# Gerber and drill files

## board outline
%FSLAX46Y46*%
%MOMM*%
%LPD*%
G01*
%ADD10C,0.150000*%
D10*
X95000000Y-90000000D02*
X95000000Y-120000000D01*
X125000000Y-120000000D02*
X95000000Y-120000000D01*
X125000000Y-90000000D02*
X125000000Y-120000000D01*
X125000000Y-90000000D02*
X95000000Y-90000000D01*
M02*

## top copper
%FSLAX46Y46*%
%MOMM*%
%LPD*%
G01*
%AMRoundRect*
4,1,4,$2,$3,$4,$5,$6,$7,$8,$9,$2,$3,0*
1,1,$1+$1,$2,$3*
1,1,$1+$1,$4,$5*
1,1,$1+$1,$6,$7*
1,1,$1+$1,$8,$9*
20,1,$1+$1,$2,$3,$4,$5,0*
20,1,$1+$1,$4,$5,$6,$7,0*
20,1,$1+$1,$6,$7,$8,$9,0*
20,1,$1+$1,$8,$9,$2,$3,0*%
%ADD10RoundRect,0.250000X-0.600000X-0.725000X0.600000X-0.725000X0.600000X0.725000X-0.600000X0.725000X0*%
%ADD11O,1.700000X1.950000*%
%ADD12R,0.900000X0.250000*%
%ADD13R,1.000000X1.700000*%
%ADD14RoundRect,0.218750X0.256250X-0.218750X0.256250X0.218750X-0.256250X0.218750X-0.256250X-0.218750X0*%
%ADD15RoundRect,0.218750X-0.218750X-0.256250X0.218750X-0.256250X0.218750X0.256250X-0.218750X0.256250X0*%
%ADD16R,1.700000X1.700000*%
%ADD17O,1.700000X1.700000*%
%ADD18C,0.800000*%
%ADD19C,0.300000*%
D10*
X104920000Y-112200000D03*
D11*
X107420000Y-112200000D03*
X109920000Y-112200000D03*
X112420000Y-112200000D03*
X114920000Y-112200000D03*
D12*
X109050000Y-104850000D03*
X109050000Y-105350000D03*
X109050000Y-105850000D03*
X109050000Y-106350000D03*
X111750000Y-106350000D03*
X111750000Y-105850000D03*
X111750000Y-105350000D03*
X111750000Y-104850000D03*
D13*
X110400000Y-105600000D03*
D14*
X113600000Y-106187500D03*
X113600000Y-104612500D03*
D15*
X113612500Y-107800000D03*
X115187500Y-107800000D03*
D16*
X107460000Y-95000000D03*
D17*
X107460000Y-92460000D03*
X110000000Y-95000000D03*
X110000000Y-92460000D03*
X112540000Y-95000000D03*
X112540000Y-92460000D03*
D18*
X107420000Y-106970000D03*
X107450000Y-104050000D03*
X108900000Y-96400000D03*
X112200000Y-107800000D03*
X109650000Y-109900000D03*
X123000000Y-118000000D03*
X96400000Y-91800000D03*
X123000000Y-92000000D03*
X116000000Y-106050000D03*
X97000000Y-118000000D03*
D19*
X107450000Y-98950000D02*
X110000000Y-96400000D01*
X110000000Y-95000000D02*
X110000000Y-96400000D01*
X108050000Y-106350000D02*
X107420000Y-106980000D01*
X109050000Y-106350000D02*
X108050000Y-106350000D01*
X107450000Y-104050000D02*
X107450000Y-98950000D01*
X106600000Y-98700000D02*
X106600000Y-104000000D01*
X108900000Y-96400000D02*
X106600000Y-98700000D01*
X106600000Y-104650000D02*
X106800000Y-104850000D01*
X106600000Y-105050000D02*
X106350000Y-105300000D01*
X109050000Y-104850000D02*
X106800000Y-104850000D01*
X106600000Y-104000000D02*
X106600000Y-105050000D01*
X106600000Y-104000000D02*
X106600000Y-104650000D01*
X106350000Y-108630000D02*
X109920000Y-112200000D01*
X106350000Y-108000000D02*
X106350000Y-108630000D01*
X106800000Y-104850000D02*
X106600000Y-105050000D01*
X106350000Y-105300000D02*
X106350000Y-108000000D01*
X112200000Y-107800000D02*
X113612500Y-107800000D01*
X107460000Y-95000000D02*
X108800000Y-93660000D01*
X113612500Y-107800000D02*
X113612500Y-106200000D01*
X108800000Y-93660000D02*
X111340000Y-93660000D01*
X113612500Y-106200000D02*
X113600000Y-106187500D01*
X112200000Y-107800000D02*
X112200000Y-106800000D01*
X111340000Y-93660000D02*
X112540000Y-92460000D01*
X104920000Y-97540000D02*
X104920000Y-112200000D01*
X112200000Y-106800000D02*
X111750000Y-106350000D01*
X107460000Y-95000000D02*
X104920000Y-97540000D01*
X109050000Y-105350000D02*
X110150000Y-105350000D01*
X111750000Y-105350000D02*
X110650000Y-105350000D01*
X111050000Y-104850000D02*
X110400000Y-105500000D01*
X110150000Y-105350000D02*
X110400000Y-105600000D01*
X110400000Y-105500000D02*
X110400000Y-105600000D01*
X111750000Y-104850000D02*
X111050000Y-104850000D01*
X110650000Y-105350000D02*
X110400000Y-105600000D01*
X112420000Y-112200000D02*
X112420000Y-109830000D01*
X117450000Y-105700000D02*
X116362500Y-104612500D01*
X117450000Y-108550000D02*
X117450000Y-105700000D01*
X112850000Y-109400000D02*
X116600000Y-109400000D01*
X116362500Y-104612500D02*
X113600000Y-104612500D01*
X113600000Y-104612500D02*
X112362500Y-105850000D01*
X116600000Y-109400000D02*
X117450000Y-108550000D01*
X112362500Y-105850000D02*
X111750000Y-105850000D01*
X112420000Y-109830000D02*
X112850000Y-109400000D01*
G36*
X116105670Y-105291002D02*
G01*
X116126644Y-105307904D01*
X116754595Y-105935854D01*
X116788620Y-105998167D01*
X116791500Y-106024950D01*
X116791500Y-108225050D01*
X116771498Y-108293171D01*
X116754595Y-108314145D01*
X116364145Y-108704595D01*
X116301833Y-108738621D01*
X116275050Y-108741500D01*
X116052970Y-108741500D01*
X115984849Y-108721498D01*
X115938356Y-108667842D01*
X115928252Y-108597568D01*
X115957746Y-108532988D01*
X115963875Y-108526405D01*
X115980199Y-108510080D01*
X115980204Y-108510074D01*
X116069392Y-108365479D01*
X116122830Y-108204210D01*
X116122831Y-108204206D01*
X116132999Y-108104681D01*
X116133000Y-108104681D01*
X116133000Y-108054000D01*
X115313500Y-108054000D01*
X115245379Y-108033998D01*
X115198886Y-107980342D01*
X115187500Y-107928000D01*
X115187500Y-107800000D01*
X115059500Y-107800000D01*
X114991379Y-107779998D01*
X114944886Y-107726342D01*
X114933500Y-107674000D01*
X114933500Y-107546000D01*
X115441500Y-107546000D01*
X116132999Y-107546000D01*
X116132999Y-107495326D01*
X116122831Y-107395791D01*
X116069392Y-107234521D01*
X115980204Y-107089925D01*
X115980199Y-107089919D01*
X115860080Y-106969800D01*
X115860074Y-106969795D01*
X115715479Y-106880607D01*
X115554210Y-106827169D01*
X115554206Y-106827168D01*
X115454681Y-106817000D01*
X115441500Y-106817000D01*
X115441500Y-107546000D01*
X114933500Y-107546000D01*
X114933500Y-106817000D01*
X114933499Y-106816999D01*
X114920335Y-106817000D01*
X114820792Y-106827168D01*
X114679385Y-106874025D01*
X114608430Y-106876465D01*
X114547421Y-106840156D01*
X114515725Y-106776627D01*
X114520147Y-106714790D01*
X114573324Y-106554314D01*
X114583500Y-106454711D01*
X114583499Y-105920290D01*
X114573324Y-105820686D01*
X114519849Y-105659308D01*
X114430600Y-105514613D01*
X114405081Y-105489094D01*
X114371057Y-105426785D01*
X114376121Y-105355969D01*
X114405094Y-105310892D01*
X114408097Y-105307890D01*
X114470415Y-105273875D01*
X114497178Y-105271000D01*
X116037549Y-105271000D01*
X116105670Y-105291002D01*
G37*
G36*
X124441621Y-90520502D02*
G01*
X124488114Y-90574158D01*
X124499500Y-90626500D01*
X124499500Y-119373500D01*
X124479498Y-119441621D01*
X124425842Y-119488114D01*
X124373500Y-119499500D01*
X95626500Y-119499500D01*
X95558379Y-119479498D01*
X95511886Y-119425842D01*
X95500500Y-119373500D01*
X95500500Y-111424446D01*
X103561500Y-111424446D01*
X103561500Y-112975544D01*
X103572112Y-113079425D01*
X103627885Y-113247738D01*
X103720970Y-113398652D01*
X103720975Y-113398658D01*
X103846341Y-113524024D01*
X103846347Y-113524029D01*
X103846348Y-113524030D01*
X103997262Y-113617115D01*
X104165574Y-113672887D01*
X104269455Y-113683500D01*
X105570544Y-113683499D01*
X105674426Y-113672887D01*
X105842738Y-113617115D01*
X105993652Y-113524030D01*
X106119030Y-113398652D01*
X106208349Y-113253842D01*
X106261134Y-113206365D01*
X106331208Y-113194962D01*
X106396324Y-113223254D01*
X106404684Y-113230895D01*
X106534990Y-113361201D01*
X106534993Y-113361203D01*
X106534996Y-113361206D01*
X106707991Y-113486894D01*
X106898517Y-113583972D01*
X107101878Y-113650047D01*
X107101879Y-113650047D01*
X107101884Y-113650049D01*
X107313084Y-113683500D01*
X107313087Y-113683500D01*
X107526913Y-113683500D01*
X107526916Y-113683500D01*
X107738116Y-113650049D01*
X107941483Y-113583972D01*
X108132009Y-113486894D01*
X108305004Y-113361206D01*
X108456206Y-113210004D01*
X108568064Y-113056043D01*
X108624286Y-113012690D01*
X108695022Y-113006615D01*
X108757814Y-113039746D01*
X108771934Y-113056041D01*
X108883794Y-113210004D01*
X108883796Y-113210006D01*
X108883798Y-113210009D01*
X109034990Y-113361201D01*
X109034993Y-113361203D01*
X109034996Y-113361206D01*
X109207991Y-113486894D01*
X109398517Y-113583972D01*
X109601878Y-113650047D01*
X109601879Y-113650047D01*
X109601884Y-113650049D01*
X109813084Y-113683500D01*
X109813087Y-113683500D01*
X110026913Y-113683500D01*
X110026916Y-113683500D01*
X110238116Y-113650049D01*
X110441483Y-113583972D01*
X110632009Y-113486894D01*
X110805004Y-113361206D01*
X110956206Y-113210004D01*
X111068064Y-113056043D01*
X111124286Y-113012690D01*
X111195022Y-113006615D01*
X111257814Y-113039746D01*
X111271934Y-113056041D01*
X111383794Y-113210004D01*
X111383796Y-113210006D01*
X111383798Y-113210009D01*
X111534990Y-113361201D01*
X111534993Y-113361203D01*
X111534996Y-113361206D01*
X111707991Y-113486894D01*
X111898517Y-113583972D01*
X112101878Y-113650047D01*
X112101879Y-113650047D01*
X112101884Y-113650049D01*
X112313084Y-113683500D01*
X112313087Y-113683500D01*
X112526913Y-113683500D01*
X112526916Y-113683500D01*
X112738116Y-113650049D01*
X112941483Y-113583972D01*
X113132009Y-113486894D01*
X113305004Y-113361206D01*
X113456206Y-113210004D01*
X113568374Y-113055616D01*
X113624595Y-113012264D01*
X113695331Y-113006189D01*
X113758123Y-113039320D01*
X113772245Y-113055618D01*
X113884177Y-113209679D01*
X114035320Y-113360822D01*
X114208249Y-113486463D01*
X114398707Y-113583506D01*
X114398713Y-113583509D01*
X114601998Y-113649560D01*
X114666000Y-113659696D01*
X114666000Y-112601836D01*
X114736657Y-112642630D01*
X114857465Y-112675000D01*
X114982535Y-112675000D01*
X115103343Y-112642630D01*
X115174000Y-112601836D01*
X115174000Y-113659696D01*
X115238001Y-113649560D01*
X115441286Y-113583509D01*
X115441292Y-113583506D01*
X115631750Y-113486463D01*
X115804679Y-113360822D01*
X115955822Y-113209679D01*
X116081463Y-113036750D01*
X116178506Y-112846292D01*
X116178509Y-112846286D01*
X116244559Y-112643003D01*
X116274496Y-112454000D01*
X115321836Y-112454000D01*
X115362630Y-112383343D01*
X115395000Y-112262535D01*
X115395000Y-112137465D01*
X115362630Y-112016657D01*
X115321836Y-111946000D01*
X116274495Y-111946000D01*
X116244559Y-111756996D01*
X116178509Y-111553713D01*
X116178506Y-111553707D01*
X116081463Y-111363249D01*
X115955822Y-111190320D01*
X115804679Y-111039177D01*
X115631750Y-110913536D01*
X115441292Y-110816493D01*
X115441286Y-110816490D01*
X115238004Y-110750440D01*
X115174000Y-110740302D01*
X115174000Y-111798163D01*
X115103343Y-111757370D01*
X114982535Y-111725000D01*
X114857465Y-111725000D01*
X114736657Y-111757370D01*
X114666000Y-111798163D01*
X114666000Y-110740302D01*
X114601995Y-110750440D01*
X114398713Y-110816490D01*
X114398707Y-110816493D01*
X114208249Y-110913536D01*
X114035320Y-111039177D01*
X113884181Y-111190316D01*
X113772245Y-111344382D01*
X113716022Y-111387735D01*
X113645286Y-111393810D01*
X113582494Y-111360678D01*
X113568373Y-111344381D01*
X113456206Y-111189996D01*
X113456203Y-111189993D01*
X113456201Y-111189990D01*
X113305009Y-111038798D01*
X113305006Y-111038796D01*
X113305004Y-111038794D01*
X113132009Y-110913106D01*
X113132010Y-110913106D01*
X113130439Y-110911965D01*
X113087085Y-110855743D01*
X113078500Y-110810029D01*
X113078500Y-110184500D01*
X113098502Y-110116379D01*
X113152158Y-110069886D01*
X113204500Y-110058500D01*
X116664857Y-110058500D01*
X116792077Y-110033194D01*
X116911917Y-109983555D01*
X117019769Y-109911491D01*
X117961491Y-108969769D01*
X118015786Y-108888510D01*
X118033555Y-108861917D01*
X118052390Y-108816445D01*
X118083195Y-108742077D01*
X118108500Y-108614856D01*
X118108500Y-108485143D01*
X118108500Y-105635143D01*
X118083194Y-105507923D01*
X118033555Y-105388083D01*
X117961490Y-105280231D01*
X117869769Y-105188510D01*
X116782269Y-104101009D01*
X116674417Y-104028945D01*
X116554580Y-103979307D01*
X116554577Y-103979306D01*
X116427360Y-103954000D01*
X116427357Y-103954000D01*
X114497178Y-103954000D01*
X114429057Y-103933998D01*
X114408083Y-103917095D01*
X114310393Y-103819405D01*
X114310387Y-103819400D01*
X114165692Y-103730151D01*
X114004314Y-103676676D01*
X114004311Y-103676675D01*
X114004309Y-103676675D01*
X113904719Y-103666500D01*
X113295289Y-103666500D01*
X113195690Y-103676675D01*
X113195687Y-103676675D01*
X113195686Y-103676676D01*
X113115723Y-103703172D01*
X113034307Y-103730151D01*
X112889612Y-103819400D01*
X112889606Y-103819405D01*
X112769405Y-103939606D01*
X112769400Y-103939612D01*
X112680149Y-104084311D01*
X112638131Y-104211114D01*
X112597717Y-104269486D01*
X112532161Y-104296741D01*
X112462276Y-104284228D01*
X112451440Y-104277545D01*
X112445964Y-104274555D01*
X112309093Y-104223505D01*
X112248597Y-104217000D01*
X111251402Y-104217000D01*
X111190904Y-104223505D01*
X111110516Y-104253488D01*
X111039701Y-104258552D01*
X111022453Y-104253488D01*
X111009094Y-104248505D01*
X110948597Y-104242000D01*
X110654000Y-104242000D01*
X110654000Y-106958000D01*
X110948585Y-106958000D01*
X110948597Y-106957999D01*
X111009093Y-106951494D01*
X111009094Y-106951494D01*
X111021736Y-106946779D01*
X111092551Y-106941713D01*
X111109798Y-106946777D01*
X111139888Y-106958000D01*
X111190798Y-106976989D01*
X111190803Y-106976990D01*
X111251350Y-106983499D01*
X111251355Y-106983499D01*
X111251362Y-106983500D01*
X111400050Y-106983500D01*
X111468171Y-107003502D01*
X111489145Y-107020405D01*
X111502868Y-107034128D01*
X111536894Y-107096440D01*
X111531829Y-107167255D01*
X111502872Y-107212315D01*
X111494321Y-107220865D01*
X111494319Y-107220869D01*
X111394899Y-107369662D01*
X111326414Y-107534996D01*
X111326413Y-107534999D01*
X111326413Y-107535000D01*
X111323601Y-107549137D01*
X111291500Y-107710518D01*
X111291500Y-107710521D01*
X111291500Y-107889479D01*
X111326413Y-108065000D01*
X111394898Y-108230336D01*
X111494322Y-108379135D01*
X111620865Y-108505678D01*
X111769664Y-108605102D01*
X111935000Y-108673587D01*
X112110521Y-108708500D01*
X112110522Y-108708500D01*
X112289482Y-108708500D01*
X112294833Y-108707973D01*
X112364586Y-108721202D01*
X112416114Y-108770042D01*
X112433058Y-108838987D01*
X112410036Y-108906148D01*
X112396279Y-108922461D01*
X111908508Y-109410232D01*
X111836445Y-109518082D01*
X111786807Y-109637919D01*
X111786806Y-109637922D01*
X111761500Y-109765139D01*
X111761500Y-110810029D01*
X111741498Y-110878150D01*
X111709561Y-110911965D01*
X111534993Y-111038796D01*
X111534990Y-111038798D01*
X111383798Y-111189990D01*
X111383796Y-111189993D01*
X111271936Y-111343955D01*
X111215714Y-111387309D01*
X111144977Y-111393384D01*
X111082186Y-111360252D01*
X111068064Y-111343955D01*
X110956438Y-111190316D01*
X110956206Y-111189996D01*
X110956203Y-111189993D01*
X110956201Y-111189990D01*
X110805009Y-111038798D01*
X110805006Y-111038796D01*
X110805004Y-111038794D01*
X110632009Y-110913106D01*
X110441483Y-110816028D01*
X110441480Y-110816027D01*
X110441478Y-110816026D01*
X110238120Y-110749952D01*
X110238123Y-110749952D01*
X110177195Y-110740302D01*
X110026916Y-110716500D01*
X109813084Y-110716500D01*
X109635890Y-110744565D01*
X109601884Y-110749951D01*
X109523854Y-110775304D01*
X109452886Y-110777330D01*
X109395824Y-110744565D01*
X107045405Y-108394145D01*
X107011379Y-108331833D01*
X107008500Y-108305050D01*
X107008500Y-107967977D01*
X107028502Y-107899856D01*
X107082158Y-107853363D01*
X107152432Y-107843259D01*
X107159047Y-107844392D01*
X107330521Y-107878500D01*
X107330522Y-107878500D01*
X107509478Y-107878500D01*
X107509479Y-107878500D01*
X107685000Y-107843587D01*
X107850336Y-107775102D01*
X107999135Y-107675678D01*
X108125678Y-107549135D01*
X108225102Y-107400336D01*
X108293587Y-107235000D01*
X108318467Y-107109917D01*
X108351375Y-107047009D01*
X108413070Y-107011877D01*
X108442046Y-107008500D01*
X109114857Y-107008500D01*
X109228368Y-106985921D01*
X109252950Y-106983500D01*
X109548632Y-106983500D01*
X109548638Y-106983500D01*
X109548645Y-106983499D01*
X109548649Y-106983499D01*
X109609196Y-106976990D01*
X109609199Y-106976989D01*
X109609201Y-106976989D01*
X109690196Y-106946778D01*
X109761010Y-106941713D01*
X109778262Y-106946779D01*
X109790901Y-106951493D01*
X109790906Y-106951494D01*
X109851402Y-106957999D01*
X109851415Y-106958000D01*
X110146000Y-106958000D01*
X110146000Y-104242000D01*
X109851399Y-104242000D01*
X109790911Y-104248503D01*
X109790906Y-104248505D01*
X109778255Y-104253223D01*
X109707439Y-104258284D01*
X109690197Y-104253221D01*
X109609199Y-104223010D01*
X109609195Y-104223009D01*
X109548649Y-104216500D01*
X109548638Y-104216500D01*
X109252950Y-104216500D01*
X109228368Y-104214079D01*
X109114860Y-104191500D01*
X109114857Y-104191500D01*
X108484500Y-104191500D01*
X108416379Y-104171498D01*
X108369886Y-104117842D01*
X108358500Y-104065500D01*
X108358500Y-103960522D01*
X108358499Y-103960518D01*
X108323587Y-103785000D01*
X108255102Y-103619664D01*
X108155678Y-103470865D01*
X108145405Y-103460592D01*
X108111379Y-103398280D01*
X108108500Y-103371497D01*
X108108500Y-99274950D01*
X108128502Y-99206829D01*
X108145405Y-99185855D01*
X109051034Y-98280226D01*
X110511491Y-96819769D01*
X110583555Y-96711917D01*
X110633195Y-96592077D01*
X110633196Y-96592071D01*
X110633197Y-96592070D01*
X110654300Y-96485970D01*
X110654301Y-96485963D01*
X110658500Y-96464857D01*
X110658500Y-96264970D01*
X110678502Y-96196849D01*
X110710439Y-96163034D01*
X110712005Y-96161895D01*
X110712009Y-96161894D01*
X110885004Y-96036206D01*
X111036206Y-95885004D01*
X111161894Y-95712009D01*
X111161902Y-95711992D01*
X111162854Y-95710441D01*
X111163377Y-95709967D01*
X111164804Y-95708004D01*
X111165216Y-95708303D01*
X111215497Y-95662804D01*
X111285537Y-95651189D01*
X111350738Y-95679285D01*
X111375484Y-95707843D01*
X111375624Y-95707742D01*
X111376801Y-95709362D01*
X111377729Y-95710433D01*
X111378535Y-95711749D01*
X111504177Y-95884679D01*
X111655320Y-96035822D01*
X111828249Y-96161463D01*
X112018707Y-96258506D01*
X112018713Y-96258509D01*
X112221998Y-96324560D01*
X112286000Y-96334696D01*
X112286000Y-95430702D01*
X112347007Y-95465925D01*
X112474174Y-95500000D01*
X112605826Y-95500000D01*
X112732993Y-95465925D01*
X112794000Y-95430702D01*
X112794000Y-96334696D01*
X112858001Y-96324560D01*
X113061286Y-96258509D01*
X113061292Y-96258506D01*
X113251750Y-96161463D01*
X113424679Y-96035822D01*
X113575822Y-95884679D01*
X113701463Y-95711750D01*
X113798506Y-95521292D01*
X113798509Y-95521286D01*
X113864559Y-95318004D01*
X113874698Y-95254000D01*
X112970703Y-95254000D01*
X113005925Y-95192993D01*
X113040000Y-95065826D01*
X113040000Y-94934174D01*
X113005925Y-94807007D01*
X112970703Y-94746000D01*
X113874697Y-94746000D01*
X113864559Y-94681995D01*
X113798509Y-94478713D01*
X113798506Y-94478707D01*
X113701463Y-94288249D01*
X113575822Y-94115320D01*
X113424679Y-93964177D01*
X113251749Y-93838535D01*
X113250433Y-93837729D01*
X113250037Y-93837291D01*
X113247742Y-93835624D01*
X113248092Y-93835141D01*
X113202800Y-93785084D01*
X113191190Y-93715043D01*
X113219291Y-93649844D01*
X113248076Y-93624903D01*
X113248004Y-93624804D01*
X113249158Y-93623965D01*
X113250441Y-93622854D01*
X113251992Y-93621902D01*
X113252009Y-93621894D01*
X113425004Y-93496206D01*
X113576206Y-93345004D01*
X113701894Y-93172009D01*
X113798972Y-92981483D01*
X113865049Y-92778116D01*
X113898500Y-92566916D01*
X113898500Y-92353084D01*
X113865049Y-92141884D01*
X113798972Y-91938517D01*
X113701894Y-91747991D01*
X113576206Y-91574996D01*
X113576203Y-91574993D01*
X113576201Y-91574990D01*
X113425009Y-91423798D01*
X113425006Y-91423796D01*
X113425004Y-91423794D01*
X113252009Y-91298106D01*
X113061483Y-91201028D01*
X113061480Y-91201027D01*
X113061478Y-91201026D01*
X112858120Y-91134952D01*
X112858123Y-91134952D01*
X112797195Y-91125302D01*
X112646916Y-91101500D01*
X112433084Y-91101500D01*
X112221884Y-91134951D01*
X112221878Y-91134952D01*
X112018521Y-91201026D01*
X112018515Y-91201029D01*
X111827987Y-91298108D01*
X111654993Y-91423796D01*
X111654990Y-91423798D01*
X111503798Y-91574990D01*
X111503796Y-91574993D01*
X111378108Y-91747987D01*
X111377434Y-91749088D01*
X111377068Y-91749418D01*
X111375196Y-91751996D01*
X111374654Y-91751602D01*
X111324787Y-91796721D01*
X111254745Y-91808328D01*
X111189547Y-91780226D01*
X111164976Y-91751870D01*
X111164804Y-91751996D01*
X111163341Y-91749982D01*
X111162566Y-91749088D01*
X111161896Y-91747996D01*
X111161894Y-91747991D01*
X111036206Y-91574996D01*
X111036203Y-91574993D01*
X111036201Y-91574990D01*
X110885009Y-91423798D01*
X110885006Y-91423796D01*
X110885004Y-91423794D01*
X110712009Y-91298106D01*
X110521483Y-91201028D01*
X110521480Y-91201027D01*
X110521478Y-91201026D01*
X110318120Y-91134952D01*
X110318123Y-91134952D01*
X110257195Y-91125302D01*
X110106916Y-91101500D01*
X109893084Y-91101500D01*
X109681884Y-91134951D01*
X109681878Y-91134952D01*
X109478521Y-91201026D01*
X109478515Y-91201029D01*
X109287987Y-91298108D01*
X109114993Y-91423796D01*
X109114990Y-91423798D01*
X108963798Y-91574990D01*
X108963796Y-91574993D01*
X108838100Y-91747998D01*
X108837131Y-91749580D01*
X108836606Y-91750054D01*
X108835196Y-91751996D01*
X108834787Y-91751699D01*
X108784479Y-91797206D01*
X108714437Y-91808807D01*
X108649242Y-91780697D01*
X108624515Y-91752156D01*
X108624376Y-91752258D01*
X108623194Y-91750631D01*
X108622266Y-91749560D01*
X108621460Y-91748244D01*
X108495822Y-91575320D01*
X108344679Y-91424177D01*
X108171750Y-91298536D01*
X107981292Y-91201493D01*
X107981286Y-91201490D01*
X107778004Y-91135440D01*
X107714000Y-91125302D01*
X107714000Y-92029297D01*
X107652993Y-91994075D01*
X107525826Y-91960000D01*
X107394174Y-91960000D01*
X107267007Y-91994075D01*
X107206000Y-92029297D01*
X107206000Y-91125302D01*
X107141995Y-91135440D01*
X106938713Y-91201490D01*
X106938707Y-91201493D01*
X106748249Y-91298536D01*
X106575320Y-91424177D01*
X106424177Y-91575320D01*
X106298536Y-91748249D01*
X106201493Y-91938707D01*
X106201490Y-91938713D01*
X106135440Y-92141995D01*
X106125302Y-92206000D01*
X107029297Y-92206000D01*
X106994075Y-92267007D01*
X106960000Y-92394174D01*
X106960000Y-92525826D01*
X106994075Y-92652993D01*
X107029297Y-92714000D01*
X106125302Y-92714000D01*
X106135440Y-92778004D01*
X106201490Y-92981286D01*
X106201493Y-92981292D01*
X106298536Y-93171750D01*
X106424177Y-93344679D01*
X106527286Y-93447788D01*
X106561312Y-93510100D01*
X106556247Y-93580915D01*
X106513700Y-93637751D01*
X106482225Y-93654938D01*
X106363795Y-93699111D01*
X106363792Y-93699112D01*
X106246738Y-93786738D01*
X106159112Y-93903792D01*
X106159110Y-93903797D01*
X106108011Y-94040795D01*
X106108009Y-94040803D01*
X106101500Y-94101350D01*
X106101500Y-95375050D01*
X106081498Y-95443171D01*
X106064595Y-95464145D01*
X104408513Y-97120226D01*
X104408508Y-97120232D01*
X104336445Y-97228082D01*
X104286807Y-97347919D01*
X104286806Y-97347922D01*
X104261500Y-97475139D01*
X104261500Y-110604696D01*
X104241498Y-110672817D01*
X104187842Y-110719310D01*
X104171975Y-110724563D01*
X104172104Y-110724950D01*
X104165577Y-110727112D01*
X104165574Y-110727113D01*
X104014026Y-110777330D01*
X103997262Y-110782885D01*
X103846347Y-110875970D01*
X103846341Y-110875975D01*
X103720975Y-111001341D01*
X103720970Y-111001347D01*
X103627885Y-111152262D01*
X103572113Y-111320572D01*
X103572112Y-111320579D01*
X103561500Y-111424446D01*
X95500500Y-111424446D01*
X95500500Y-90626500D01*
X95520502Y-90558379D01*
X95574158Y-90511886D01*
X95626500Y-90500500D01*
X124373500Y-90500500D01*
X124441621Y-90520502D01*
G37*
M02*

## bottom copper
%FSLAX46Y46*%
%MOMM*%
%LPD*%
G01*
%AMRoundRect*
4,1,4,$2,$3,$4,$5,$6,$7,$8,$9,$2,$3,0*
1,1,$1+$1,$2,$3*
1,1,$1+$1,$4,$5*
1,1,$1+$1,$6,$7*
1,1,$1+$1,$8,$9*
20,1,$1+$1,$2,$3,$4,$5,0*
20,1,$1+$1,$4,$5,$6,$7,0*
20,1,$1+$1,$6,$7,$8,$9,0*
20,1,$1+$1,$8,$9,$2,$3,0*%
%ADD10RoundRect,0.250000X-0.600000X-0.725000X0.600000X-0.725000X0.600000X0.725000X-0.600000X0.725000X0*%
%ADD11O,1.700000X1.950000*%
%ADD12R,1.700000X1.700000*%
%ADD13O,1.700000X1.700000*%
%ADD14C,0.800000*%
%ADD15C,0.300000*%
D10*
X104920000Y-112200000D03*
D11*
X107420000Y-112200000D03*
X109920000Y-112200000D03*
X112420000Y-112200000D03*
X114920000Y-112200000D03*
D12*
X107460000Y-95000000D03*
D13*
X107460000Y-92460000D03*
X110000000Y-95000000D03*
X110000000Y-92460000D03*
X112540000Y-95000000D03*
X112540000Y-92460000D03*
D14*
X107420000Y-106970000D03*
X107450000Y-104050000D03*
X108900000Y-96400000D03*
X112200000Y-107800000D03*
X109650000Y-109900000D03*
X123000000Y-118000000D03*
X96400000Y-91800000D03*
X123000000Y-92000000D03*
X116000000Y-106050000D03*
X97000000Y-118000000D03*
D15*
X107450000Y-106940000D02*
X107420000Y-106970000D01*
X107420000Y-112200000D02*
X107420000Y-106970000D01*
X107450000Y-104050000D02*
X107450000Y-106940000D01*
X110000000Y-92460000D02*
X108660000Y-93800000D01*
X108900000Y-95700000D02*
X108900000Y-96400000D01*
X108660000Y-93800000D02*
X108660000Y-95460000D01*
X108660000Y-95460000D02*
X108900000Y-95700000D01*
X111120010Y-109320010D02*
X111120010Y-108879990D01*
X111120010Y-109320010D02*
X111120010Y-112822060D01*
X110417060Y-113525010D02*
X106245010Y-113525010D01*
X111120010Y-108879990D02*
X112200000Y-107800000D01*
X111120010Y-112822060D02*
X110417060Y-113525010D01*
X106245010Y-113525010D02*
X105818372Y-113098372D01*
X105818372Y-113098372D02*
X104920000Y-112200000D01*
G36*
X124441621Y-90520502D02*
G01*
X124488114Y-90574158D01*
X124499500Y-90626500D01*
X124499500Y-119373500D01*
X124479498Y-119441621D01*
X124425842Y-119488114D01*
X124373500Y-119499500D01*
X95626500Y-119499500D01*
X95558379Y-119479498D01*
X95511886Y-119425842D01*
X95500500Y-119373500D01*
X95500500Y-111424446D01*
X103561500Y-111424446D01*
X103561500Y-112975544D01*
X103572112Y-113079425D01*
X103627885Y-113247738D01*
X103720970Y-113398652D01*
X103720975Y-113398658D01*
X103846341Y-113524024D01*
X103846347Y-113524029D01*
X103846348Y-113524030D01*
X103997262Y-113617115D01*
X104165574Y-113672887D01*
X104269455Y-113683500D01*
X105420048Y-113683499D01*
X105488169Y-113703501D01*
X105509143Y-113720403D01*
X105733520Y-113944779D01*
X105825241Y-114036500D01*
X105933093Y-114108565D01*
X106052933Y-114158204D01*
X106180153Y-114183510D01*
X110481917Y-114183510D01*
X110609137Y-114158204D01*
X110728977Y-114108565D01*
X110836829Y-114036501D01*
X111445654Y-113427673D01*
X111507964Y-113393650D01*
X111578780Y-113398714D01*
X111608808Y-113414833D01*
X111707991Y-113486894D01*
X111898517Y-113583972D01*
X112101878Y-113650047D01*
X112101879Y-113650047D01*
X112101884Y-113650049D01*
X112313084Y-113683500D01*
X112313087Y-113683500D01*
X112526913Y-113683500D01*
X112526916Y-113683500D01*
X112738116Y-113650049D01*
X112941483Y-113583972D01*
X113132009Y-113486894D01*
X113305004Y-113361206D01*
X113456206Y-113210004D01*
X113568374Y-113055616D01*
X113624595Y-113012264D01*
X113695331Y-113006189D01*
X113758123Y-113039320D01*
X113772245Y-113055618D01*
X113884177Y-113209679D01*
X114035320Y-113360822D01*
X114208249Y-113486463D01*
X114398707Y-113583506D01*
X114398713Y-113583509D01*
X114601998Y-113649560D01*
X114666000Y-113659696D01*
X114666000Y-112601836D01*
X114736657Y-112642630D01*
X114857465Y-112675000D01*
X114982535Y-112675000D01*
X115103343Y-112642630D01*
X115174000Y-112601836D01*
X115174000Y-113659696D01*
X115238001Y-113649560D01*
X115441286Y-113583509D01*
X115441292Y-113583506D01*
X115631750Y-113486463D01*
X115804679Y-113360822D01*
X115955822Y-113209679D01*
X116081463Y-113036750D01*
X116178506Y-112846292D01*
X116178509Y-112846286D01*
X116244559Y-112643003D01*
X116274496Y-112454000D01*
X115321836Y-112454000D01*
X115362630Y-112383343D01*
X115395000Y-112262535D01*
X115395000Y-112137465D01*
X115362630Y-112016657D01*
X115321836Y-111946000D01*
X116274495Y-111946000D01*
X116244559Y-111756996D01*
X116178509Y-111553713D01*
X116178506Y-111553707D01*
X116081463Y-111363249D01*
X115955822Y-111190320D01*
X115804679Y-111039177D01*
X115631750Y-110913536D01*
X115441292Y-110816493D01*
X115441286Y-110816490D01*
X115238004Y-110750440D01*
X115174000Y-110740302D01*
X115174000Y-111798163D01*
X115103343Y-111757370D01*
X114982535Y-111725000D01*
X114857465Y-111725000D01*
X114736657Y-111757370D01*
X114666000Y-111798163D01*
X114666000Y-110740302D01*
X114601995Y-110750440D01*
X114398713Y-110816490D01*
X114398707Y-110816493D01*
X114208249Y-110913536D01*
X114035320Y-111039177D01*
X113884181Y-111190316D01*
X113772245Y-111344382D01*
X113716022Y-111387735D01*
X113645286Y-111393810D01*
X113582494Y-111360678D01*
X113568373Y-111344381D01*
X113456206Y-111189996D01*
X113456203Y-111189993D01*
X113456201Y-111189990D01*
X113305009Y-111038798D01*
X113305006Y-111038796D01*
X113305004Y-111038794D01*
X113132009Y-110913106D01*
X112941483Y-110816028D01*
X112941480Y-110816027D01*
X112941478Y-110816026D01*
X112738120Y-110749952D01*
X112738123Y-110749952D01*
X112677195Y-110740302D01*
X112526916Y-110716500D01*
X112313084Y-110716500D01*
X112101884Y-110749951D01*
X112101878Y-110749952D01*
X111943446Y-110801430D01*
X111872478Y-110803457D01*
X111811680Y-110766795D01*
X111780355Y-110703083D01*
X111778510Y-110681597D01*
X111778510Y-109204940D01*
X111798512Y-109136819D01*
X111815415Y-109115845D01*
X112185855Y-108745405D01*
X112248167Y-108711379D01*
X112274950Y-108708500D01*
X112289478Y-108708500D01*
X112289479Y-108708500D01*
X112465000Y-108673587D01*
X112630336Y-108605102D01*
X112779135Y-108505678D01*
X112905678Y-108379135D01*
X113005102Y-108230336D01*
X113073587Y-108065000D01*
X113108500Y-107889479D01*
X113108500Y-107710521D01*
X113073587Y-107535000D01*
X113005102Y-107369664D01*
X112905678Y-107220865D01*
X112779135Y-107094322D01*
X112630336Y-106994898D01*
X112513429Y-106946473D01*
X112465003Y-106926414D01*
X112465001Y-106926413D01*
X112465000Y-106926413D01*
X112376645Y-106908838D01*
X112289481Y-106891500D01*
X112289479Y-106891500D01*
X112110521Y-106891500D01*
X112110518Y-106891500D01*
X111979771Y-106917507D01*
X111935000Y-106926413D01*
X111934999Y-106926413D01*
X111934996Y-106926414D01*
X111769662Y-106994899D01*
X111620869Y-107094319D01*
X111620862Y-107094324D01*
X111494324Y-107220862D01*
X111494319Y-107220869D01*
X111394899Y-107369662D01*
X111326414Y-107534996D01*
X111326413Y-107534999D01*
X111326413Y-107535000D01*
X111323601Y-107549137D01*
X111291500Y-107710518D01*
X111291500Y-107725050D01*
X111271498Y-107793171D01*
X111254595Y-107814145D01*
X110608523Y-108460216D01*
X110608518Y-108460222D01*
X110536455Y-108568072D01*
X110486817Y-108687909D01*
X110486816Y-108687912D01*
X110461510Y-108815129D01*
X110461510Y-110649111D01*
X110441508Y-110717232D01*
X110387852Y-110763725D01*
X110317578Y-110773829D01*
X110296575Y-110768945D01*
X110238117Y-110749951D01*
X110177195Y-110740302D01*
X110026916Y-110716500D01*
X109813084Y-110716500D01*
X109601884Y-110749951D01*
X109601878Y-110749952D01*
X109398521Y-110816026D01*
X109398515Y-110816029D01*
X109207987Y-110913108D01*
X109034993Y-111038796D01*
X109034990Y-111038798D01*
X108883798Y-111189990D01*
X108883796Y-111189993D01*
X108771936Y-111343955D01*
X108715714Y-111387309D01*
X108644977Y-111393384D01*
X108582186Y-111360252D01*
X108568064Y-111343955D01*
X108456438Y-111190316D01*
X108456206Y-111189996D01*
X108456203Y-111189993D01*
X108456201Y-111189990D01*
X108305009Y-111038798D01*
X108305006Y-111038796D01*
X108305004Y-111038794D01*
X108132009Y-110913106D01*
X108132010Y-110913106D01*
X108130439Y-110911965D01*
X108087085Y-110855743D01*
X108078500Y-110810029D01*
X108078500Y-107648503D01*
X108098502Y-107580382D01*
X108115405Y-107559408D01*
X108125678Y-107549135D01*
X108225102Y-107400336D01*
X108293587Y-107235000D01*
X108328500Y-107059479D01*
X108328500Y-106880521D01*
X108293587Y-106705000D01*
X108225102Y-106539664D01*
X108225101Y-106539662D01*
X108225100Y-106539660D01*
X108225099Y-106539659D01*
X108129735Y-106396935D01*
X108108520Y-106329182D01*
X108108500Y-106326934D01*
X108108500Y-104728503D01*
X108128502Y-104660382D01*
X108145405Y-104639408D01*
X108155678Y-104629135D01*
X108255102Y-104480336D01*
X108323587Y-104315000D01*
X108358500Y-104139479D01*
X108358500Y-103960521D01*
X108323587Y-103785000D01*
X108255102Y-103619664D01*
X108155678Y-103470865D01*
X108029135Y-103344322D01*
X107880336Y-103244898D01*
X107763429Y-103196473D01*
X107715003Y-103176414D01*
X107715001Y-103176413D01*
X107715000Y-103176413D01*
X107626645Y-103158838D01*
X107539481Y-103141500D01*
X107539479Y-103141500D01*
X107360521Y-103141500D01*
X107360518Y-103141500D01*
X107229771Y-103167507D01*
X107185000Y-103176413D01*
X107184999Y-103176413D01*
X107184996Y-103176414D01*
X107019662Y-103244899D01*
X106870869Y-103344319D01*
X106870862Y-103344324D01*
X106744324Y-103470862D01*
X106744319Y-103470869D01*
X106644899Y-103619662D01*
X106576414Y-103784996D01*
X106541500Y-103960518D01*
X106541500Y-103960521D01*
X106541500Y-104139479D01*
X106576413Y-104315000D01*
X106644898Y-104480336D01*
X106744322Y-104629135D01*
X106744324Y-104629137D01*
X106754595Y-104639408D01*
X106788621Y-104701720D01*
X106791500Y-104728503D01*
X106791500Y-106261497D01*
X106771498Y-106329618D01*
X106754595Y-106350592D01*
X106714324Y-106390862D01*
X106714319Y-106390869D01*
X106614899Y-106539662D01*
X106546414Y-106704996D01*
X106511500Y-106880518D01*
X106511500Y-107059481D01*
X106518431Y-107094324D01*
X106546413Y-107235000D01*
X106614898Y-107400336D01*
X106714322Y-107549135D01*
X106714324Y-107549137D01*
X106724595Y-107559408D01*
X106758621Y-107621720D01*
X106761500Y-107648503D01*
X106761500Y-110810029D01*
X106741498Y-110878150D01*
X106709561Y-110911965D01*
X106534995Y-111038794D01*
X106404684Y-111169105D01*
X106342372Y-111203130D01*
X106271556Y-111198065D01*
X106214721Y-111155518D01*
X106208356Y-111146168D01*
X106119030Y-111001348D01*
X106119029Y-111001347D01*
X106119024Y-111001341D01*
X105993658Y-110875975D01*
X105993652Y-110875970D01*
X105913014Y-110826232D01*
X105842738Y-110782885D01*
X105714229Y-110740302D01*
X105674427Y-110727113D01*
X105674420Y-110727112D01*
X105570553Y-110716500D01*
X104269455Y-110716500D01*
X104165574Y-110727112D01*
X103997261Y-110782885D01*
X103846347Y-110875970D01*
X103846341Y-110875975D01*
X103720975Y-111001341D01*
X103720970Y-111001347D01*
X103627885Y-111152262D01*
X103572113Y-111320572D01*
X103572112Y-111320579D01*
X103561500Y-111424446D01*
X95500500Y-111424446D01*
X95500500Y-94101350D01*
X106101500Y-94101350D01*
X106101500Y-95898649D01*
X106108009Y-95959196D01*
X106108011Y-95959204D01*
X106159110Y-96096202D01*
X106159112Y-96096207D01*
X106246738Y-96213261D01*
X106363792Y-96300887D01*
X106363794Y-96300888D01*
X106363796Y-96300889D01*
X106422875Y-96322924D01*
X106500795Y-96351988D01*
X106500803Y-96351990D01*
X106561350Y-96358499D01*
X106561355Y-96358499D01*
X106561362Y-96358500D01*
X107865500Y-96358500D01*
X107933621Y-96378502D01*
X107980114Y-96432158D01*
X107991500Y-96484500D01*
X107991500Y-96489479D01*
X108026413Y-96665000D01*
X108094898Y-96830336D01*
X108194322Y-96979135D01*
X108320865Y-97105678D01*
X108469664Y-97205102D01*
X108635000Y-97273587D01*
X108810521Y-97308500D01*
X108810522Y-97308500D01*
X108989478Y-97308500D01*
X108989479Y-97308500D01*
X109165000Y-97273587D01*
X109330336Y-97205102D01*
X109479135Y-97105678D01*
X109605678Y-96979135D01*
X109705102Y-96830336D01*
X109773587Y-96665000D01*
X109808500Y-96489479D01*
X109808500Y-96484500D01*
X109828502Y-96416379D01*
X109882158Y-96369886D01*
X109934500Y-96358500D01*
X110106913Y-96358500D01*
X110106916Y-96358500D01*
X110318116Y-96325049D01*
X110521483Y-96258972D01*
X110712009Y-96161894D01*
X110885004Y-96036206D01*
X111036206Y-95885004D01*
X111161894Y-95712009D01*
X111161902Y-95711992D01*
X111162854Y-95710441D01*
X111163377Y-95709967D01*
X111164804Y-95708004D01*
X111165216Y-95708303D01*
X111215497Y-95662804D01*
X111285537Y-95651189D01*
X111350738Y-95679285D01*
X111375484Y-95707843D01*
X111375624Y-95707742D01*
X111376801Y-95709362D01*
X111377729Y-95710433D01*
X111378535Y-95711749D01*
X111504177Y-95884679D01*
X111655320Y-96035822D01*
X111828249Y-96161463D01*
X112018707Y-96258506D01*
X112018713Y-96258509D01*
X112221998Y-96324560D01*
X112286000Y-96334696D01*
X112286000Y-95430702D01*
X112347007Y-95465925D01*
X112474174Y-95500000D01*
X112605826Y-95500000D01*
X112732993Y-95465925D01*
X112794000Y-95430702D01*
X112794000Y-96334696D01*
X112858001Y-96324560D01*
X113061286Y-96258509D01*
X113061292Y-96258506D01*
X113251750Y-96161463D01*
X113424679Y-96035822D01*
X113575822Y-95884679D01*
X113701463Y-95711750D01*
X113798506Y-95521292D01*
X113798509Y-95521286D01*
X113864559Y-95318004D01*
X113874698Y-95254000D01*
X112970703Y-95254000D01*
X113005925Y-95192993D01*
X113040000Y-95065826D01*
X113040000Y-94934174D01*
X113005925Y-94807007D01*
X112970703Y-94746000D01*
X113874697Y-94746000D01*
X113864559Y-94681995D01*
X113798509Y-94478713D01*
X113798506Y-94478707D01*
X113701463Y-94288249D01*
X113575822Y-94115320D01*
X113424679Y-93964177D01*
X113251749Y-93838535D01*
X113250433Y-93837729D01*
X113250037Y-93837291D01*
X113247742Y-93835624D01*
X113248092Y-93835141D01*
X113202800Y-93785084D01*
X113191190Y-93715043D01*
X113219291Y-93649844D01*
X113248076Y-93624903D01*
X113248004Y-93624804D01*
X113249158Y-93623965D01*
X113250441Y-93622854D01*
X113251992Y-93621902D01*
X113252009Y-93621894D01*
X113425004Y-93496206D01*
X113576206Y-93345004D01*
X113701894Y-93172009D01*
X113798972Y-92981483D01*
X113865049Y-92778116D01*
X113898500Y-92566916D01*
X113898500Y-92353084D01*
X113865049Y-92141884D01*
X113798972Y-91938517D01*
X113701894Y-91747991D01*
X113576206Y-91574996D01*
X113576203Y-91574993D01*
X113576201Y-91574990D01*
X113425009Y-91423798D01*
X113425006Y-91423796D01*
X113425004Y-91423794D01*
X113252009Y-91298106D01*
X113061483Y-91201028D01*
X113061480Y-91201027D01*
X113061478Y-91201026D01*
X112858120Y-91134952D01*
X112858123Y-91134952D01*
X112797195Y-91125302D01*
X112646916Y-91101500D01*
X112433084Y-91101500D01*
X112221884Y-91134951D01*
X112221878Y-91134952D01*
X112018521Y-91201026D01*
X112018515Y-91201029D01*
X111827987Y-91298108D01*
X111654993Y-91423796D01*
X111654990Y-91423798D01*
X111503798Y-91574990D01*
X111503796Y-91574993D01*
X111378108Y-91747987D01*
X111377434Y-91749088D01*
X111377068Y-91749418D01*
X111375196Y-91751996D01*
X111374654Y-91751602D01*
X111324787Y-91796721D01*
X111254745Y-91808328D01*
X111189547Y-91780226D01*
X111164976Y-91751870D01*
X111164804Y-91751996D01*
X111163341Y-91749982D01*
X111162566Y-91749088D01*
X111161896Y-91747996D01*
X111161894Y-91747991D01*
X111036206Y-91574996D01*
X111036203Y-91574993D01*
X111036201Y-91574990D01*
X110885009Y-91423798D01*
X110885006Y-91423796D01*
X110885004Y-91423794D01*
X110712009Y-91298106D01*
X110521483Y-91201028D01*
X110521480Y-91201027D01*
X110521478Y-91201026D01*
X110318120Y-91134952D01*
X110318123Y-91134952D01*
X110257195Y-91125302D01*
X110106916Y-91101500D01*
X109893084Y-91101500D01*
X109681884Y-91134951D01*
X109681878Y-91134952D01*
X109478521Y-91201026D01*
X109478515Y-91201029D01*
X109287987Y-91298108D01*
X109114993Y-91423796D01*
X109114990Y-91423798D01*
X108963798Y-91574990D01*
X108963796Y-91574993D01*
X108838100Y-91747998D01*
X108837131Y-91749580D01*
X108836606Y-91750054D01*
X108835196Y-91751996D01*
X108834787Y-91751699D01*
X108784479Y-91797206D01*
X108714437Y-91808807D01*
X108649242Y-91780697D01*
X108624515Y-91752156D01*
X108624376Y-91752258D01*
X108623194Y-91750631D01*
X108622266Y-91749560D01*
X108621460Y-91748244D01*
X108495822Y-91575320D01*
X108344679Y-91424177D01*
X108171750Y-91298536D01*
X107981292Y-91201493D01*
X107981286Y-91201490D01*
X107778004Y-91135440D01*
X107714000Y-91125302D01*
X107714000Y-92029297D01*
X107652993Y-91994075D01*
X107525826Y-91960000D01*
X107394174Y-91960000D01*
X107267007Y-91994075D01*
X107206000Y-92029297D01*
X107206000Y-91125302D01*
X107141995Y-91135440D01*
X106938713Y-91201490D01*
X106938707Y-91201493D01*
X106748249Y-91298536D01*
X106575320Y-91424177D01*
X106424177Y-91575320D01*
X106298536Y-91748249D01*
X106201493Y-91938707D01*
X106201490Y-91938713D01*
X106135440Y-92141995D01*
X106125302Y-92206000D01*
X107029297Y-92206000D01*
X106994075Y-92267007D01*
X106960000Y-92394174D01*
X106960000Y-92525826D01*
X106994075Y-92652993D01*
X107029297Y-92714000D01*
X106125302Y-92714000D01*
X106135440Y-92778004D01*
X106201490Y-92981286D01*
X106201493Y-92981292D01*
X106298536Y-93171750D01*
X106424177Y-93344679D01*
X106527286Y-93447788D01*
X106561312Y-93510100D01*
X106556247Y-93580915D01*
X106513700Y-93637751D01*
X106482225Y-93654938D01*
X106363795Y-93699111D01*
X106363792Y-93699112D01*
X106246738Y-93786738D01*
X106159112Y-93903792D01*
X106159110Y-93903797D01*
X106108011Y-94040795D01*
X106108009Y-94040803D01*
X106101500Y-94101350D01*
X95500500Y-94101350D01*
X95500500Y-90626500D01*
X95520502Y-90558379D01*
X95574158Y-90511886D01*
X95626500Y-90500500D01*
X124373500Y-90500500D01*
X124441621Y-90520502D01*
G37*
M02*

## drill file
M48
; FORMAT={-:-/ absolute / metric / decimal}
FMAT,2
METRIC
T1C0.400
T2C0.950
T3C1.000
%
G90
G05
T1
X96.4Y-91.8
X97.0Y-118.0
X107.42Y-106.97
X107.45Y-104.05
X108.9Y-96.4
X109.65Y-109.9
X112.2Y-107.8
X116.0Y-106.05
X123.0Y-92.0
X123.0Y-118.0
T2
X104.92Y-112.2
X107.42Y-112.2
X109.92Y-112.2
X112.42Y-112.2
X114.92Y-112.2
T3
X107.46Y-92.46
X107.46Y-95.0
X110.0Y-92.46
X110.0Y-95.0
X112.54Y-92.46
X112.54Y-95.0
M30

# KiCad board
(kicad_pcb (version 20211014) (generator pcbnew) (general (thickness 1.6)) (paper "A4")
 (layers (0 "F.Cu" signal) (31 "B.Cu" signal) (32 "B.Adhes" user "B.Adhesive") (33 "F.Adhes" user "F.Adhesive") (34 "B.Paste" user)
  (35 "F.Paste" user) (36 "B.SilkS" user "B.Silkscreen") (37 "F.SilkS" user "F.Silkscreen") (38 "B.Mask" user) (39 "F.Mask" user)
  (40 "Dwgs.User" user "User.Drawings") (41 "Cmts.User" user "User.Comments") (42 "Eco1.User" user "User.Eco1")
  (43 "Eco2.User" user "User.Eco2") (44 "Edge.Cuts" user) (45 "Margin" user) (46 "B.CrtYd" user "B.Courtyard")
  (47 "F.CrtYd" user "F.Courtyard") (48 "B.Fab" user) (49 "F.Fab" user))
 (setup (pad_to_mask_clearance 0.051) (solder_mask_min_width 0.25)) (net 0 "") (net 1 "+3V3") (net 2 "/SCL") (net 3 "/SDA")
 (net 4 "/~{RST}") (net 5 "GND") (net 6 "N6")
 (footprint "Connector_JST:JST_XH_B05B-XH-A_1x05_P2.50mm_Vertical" (layer "F.Cu") (at 104.92 112.2)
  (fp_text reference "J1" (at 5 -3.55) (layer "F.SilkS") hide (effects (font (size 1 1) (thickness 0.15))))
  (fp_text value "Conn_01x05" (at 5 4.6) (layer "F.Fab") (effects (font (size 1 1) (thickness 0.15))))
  (pad "1" thru_hole roundrect locked (at 0 0) (size 1.7 1.95) (drill 0.95) (layers *.Cu *.Mask) (roundrect_rratio 0.147059) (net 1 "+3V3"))
  (pad "2" thru_hole oval locked (at 2.5 0) (size 1.7 1.95) (drill 0.95) (layers *.Cu *.Mask) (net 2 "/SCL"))
  (pad "3" thru_hole oval locked (at 5 0) (size 1.7 1.95) (drill 0.95) (layers *.Cu *.Mask) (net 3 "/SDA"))
  (pad "4" thru_hole oval locked (at 7.5 0) (size 1.7 1.95) (drill 0.95) (layers *.Cu *.Mask) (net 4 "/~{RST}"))
  (pad "5" thru_hole oval locked (at 10 0) (size 1.7 1.95) (drill 0.95) (layers *.Cu *.Mask) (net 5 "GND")))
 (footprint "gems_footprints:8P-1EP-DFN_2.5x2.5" (layer "F.Cu") (at 110.4 105.6)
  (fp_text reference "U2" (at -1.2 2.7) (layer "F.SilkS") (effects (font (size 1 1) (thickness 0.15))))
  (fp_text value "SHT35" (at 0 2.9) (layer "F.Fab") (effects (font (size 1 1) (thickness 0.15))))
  (pad "1" smd rect locked (at -1.35 -0.75) (size 0.9 0.25) (layers "F.Cu" "F.Paste" "F.Mask") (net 3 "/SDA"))
  (pad "2" smd rect locked (at -1.35 -0.25) (size 0.9 0.25) (layers "F.Cu" "F.Paste" "F.Mask") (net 5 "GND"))
  (pad "3" smd rect locked (at -1.35 0.25) (size 0.9 0.25) (layers "F.Cu" "F.Paste" "F.Mask") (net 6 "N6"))
  (pad "4" smd rect locked (at -1.35 0.75) (size 0.9 0.25) (layers "F.Cu" "F.Paste" "F.Mask") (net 2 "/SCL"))
  (pad "5" smd rect locked (at 1.35 0.75) (size 0.9 0.25) (layers "F.Cu" "F.Paste" "F.Mask") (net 1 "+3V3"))
  (pad "6" smd rect locked (at 1.35 0.25) (size 0.9 0.25) (layers "F.Cu" "F.Paste" "F.Mask") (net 4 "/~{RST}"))
  (pad "7" smd rect locked (at 1.35 -0.25) (size 0.9 0.25) (layers "F.Cu" "F.Paste" "F.Mask") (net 5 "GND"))
  (pad "8" smd rect locked (at 1.35 -0.75) (size 0.9 0.25) (layers "F.Cu" "F.Paste" "F.Mask") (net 5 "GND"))
  (pad "9" smd rect locked (at 0 0) (size 1 1.7) (layers "F.Cu" "F.Mask") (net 5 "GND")))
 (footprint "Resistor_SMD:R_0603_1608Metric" (layer "F.Cu") (at 113.6 105.4 90)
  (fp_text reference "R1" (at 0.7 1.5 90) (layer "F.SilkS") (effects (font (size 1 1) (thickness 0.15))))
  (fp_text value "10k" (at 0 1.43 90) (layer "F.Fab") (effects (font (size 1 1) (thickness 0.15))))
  (pad "1" smd roundrect locked (at -0.7875 0 90) (size 0.875 0.95) (layers "F.Cu" "F.Paste" "F.Mask") (roundrect_rratio 0.25)
   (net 1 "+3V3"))
  (pad "2" smd roundrect locked (at 0.7875 0 90) (size 0.875 0.95) (layers "F.Cu" "F.Paste" "F.Mask") (roundrect_rratio 0.25)
   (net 4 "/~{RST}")))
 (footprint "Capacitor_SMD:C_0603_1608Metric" (layer "F.Cu") (at 114.4 107.8)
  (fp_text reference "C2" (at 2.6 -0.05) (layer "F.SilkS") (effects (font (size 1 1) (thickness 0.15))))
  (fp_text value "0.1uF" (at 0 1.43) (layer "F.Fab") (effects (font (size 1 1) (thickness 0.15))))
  (pad "1" smd roundrect locked (at -0.7875 0) (size 0.875 0.95) (layers "F.Cu" "F.Paste" "F.Mask") (roundrect_rratio 0.25) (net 1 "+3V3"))
  (pad "2" smd roundrect locked (at 0.7875 0) (size 0.875 0.95) (layers "F.Cu" "F.Paste" "F.Mask") (roundrect_rratio 0.25) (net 5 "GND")))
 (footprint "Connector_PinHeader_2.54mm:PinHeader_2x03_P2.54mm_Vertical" (layer "F.Cu") (at 107.46 95 90)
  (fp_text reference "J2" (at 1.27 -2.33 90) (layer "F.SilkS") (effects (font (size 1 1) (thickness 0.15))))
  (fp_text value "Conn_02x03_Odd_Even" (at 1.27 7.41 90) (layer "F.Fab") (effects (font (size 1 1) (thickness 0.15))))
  (pad "1" thru_hole rect (at 0 0 90) (size 1.7 1.7) (drill 1) (layers *.Cu *.Mask) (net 1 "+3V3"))
  (pad "2" thru_hole oval (at 2.54 0 90) (size 1.7 1.7) (drill 1) (layers *.Cu *.Mask) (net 5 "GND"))
  (pad "3" thru_hole oval (at 0 2.54 90) (size 1.7 1.7) (drill 1) (layers *.Cu *.Mask) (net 2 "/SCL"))
  (pad "4" thru_hole oval (at 2.54 2.54 90) (size 1.7 1.7) (drill 1) (layers *.Cu *.Mask) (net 3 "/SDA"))
  (pad "5" thru_hole oval (at 0 5.08 90) (size 1.7 1.7) (drill 1) (layers *.Cu *.Mask) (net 5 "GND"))
  (pad "6" thru_hole oval (at 2.54 5.08 90) (size 1.7 1.7) (drill 1) (layers *.Cu *.Mask) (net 1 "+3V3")))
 (gr_line (start 95 90) (end 95 120) (layer "Edge.Cuts") (width 0.15))
 (gr_line (start 125 120) (end 95 120) (layer "Edge.Cuts") (width 0.15))
 (gr_line (start 125 90) (end 125 120) (layer "Edge.Cuts") (width 0.15))
 (gr_line (start 125 90) (end 95 90) (layer "Edge.Cuts") (width 0.15))
 (segment (start 107.45 98.95) (end 110 96.4) (width 0.3) (layer "F.Cu") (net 2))
 (segment (start 110 95) (end 110 96.4) (width 0.3) (layer "F.Cu") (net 2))
 (segment (start 108.05 106.35) (end 107.42 106.98) (width 0.3) (layer "F.Cu") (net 2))
 (segment (start 109.05 106.35) (end 108.05 106.35) (width 0.3) (layer "F.Cu") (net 2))
 (segment (start 107.45 104.05) (end 107.45 98.95) (width 0.3) (layer "F.Cu") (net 2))
 (via (at 107.42 106.97) (size 0.8) (drill 0.4) (layers "F.Cu" "B.Cu") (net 2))
 (via (at 107.45 104.05) (size 0.8) (drill 0.4) (layers "F.Cu" "B.Cu") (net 2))
 (segment (start 107.45 106.94) (end 107.42 106.97) (width 0.3) (layer "B.Cu") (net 2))
 (segment (start 107.42 112.2) (end 107.42 106.97) (width 0.3) (layer "B.Cu") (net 2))
 (segment (start 107.45 104.05) (end 107.45 106.94) (width 0.3) (layer "B.Cu") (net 2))
 (segment (start 106.6 98.7) (end 106.6 104) (width 0.3) (layer "F.Cu") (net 3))
 (segment (start 108.9 96.4) (end 106.6 98.7) (width 0.3) (layer "F.Cu") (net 3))
 (segment (start 106.6 104.65) (end 106.8 104.85) (width 0.3) (layer "F.Cu") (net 3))
 (segment (start 106.6 105.05) (end 106.35 105.3) (width 0.3) (layer "F.Cu") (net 3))
 (segment (start 109.05 104.85) (end 106.8 104.85) (width 0.3) (layer "F.Cu") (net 3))
 (segment (start 106.6 104) (end 106.6 105.05) (width 0.3) (layer "F.Cu") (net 3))
 (segment (start 106.6 104) (end 106.6 104.65) (width 0.3) (layer "F.Cu") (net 3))
 (segment (start 106.35 108.63) (end 109.92 112.2) (width 0.3) (layer "F.Cu") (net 3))
 (segment (start 106.35 108) (end 106.35 108.63) (width 0.3) (layer "F.Cu") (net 3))
 (segment (start 106.8 104.85) (end 106.6 105.05) (width 0.3) (layer "F.Cu") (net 3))
 (segment (start 106.35 105.3) (end 106.35 108) (width 0.3) (layer "F.Cu") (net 3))
 (via (at 108.9 96.4) (size 0.8) (drill 0.4) (layers "F.Cu" "B.Cu") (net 3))
 (segment (start 110 92.46) (end 108.66 93.8) (width 0.3) (layer "B.Cu") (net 3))
 (segment (start 108.9 95.7) (end 108.9 96.4) (width 0.3) (layer "B.Cu") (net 3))
 (segment (start 108.66 93.8) (end 108.66 95.46) (width 0.3) (layer "B.Cu") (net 3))
 (segment (start 108.66 95.46) (end 108.9 95.7) (width 0.3) (layer "B.Cu") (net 3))
 (segment (start 112.2 107.8) (end 113.6125 107.8) (width 0.3) (layer "F.Cu") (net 1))
 (segment (start 107.46 95) (end 108.8 93.66) (width 0.3) (layer "F.Cu") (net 1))
 (segment (start 113.6125 107.8) (end 113.6125 106.2) (width 0.3) (layer "F.Cu") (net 1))
 (segment (start 108.8 93.66) (end 111.34 93.66) (width 0.3) (layer "F.Cu") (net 1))
 (segment (start 113.6125 106.2) (end 113.6 106.1875) (width 0.3) (layer "F.Cu") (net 1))
 (segment (start 112.2 107.8) (end 112.2 106.8) (width 0.3) (layer "F.Cu") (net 1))
 (segment (start 111.34 93.66) (end 112.54 92.46) (width 0.3) (layer "F.Cu") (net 1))
 (segment (start 104.92 97.54) (end 104.92 112.2) (width 0.3) (layer "F.Cu") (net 1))
 (segment (start 112.2 106.8) (end 111.75 106.35) (width 0.3) (layer "F.Cu") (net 1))
 (segment (start 107.46 95) (end 104.92 97.54) (width 0.3) (layer "F.Cu") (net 1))
 (via (at 112.2 107.8) (size 0.8) (drill 0.4) (layers "F.Cu" "B.Cu") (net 1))
 (segment (start 111.12001 109.32001) (end 111.12001 108.87999) (width 0.3) (layer "B.Cu") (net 1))
 (segment (start 111.12001 109.32001) (end 111.12001 112.82206) (width 0.3) (layer "B.Cu") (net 1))
 (segment (start 110.41706 113.52501) (end 106.24501 113.52501) (width 0.3) (layer "B.Cu") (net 1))
 (segment (start 111.12001 108.87999) (end 112.2 107.8) (width 0.3) (layer "B.Cu") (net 1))
 (segment (start 111.12001 112.82206) (end 110.41706 113.52501) (width 0.3) (layer "B.Cu") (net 1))
 (segment (start 106.24501 113.52501) (end 105.818372 113.098372) (width 0.3) (layer "B.Cu") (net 1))
 (segment (start 105.818372 113.098372) (end 104.92 112.2) (width 0.3) (layer "B.Cu") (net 1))
 (segment (start 109.05 105.35) (end 110.15 105.35) (width 0.3) (layer "F.Cu") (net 5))
 (segment (start 111.75 105.35) (end 110.65 105.35) (width 0.3) (layer "F.Cu") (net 5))
 (segment (start 111.05 104.85) (end 110.4 105.5) (width 0.3) (layer "F.Cu") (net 5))
 (segment (start 110.15 105.35) (end 110.4 105.6) (width 0.3) (layer "F.Cu") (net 5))
 (segment (start 110.4 105.5) (end 110.4 105.6) (width 0.3) (layer "F.Cu") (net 5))
 (segment (start 111.75 104.85) (end 111.05 104.85) (width 0.3) (layer "F.Cu") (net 5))
 (segment (start 110.65 105.35) (end 110.4 105.6) (width 0.3) (layer "F.Cu") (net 5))
 (via (at 109.65 109.9) (size 0.8) (drill 0.4) (layers "F.Cu" "B.Cu") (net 5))
 (via (at 123 118) (size 0.8) (drill 0.4) (layers "F.Cu" "B.Cu") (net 5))
 (via (at 96.4 91.8) (size 0.8) (drill 0.4) (layers "F.Cu" "B.Cu") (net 5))
 (via (at 123 92) (size 0.8) (drill 0.4) (layers "F.Cu" "B.Cu") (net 5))
 (via (at 116 106.05) (size 0.8) (drill 0.4) (layers "F.Cu" "B.Cu") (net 5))
 (via (at 97 118) (size 0.8) (drill 0.4) (layers "F.Cu" "B.Cu") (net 5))
 (segment (start 112.42 112.2) (end 112.42 109.83) (width 0.3) (layer "F.Cu") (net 4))
 (segment (start 117.45 105.7) (end 116.3625 104.6125) (width 0.3) (layer "F.Cu") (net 4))
 (segment (start 117.45 108.55) (end 117.45 105.7) (width 0.3) (layer "F.Cu") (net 4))
 (segment (start 112.85 109.4) (end 116.6 109.4) (width 0.3) (layer "F.Cu") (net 4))
 (segment (start 116.3625 104.6125) (end 113.6 104.6125) (width 0.3) (layer "F.Cu") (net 4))
 (segment (start 113.6 104.6125) (end 112.3625 105.85) (width 0.3) (layer "F.Cu") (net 4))
 (segment (start 116.6 109.4) (end 117.45 108.55) (width 0.3) (layer "F.Cu") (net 4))
 (segment (start 112.3625 105.85) (end 111.75 105.85) (width 0.3) (layer "F.Cu") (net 4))
 (segment (start 112.42 109.83) (end 112.85 109.4) (width 0.3) (layer "F.Cu") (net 4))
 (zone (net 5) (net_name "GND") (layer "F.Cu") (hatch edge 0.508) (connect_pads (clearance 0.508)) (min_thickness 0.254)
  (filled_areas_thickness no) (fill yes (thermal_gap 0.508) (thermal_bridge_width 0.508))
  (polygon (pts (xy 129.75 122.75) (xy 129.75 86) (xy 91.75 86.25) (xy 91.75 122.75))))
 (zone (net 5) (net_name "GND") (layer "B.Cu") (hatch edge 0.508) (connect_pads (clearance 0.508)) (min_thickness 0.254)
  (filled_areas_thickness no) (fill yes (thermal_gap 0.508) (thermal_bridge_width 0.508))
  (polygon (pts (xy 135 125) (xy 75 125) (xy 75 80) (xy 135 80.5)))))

